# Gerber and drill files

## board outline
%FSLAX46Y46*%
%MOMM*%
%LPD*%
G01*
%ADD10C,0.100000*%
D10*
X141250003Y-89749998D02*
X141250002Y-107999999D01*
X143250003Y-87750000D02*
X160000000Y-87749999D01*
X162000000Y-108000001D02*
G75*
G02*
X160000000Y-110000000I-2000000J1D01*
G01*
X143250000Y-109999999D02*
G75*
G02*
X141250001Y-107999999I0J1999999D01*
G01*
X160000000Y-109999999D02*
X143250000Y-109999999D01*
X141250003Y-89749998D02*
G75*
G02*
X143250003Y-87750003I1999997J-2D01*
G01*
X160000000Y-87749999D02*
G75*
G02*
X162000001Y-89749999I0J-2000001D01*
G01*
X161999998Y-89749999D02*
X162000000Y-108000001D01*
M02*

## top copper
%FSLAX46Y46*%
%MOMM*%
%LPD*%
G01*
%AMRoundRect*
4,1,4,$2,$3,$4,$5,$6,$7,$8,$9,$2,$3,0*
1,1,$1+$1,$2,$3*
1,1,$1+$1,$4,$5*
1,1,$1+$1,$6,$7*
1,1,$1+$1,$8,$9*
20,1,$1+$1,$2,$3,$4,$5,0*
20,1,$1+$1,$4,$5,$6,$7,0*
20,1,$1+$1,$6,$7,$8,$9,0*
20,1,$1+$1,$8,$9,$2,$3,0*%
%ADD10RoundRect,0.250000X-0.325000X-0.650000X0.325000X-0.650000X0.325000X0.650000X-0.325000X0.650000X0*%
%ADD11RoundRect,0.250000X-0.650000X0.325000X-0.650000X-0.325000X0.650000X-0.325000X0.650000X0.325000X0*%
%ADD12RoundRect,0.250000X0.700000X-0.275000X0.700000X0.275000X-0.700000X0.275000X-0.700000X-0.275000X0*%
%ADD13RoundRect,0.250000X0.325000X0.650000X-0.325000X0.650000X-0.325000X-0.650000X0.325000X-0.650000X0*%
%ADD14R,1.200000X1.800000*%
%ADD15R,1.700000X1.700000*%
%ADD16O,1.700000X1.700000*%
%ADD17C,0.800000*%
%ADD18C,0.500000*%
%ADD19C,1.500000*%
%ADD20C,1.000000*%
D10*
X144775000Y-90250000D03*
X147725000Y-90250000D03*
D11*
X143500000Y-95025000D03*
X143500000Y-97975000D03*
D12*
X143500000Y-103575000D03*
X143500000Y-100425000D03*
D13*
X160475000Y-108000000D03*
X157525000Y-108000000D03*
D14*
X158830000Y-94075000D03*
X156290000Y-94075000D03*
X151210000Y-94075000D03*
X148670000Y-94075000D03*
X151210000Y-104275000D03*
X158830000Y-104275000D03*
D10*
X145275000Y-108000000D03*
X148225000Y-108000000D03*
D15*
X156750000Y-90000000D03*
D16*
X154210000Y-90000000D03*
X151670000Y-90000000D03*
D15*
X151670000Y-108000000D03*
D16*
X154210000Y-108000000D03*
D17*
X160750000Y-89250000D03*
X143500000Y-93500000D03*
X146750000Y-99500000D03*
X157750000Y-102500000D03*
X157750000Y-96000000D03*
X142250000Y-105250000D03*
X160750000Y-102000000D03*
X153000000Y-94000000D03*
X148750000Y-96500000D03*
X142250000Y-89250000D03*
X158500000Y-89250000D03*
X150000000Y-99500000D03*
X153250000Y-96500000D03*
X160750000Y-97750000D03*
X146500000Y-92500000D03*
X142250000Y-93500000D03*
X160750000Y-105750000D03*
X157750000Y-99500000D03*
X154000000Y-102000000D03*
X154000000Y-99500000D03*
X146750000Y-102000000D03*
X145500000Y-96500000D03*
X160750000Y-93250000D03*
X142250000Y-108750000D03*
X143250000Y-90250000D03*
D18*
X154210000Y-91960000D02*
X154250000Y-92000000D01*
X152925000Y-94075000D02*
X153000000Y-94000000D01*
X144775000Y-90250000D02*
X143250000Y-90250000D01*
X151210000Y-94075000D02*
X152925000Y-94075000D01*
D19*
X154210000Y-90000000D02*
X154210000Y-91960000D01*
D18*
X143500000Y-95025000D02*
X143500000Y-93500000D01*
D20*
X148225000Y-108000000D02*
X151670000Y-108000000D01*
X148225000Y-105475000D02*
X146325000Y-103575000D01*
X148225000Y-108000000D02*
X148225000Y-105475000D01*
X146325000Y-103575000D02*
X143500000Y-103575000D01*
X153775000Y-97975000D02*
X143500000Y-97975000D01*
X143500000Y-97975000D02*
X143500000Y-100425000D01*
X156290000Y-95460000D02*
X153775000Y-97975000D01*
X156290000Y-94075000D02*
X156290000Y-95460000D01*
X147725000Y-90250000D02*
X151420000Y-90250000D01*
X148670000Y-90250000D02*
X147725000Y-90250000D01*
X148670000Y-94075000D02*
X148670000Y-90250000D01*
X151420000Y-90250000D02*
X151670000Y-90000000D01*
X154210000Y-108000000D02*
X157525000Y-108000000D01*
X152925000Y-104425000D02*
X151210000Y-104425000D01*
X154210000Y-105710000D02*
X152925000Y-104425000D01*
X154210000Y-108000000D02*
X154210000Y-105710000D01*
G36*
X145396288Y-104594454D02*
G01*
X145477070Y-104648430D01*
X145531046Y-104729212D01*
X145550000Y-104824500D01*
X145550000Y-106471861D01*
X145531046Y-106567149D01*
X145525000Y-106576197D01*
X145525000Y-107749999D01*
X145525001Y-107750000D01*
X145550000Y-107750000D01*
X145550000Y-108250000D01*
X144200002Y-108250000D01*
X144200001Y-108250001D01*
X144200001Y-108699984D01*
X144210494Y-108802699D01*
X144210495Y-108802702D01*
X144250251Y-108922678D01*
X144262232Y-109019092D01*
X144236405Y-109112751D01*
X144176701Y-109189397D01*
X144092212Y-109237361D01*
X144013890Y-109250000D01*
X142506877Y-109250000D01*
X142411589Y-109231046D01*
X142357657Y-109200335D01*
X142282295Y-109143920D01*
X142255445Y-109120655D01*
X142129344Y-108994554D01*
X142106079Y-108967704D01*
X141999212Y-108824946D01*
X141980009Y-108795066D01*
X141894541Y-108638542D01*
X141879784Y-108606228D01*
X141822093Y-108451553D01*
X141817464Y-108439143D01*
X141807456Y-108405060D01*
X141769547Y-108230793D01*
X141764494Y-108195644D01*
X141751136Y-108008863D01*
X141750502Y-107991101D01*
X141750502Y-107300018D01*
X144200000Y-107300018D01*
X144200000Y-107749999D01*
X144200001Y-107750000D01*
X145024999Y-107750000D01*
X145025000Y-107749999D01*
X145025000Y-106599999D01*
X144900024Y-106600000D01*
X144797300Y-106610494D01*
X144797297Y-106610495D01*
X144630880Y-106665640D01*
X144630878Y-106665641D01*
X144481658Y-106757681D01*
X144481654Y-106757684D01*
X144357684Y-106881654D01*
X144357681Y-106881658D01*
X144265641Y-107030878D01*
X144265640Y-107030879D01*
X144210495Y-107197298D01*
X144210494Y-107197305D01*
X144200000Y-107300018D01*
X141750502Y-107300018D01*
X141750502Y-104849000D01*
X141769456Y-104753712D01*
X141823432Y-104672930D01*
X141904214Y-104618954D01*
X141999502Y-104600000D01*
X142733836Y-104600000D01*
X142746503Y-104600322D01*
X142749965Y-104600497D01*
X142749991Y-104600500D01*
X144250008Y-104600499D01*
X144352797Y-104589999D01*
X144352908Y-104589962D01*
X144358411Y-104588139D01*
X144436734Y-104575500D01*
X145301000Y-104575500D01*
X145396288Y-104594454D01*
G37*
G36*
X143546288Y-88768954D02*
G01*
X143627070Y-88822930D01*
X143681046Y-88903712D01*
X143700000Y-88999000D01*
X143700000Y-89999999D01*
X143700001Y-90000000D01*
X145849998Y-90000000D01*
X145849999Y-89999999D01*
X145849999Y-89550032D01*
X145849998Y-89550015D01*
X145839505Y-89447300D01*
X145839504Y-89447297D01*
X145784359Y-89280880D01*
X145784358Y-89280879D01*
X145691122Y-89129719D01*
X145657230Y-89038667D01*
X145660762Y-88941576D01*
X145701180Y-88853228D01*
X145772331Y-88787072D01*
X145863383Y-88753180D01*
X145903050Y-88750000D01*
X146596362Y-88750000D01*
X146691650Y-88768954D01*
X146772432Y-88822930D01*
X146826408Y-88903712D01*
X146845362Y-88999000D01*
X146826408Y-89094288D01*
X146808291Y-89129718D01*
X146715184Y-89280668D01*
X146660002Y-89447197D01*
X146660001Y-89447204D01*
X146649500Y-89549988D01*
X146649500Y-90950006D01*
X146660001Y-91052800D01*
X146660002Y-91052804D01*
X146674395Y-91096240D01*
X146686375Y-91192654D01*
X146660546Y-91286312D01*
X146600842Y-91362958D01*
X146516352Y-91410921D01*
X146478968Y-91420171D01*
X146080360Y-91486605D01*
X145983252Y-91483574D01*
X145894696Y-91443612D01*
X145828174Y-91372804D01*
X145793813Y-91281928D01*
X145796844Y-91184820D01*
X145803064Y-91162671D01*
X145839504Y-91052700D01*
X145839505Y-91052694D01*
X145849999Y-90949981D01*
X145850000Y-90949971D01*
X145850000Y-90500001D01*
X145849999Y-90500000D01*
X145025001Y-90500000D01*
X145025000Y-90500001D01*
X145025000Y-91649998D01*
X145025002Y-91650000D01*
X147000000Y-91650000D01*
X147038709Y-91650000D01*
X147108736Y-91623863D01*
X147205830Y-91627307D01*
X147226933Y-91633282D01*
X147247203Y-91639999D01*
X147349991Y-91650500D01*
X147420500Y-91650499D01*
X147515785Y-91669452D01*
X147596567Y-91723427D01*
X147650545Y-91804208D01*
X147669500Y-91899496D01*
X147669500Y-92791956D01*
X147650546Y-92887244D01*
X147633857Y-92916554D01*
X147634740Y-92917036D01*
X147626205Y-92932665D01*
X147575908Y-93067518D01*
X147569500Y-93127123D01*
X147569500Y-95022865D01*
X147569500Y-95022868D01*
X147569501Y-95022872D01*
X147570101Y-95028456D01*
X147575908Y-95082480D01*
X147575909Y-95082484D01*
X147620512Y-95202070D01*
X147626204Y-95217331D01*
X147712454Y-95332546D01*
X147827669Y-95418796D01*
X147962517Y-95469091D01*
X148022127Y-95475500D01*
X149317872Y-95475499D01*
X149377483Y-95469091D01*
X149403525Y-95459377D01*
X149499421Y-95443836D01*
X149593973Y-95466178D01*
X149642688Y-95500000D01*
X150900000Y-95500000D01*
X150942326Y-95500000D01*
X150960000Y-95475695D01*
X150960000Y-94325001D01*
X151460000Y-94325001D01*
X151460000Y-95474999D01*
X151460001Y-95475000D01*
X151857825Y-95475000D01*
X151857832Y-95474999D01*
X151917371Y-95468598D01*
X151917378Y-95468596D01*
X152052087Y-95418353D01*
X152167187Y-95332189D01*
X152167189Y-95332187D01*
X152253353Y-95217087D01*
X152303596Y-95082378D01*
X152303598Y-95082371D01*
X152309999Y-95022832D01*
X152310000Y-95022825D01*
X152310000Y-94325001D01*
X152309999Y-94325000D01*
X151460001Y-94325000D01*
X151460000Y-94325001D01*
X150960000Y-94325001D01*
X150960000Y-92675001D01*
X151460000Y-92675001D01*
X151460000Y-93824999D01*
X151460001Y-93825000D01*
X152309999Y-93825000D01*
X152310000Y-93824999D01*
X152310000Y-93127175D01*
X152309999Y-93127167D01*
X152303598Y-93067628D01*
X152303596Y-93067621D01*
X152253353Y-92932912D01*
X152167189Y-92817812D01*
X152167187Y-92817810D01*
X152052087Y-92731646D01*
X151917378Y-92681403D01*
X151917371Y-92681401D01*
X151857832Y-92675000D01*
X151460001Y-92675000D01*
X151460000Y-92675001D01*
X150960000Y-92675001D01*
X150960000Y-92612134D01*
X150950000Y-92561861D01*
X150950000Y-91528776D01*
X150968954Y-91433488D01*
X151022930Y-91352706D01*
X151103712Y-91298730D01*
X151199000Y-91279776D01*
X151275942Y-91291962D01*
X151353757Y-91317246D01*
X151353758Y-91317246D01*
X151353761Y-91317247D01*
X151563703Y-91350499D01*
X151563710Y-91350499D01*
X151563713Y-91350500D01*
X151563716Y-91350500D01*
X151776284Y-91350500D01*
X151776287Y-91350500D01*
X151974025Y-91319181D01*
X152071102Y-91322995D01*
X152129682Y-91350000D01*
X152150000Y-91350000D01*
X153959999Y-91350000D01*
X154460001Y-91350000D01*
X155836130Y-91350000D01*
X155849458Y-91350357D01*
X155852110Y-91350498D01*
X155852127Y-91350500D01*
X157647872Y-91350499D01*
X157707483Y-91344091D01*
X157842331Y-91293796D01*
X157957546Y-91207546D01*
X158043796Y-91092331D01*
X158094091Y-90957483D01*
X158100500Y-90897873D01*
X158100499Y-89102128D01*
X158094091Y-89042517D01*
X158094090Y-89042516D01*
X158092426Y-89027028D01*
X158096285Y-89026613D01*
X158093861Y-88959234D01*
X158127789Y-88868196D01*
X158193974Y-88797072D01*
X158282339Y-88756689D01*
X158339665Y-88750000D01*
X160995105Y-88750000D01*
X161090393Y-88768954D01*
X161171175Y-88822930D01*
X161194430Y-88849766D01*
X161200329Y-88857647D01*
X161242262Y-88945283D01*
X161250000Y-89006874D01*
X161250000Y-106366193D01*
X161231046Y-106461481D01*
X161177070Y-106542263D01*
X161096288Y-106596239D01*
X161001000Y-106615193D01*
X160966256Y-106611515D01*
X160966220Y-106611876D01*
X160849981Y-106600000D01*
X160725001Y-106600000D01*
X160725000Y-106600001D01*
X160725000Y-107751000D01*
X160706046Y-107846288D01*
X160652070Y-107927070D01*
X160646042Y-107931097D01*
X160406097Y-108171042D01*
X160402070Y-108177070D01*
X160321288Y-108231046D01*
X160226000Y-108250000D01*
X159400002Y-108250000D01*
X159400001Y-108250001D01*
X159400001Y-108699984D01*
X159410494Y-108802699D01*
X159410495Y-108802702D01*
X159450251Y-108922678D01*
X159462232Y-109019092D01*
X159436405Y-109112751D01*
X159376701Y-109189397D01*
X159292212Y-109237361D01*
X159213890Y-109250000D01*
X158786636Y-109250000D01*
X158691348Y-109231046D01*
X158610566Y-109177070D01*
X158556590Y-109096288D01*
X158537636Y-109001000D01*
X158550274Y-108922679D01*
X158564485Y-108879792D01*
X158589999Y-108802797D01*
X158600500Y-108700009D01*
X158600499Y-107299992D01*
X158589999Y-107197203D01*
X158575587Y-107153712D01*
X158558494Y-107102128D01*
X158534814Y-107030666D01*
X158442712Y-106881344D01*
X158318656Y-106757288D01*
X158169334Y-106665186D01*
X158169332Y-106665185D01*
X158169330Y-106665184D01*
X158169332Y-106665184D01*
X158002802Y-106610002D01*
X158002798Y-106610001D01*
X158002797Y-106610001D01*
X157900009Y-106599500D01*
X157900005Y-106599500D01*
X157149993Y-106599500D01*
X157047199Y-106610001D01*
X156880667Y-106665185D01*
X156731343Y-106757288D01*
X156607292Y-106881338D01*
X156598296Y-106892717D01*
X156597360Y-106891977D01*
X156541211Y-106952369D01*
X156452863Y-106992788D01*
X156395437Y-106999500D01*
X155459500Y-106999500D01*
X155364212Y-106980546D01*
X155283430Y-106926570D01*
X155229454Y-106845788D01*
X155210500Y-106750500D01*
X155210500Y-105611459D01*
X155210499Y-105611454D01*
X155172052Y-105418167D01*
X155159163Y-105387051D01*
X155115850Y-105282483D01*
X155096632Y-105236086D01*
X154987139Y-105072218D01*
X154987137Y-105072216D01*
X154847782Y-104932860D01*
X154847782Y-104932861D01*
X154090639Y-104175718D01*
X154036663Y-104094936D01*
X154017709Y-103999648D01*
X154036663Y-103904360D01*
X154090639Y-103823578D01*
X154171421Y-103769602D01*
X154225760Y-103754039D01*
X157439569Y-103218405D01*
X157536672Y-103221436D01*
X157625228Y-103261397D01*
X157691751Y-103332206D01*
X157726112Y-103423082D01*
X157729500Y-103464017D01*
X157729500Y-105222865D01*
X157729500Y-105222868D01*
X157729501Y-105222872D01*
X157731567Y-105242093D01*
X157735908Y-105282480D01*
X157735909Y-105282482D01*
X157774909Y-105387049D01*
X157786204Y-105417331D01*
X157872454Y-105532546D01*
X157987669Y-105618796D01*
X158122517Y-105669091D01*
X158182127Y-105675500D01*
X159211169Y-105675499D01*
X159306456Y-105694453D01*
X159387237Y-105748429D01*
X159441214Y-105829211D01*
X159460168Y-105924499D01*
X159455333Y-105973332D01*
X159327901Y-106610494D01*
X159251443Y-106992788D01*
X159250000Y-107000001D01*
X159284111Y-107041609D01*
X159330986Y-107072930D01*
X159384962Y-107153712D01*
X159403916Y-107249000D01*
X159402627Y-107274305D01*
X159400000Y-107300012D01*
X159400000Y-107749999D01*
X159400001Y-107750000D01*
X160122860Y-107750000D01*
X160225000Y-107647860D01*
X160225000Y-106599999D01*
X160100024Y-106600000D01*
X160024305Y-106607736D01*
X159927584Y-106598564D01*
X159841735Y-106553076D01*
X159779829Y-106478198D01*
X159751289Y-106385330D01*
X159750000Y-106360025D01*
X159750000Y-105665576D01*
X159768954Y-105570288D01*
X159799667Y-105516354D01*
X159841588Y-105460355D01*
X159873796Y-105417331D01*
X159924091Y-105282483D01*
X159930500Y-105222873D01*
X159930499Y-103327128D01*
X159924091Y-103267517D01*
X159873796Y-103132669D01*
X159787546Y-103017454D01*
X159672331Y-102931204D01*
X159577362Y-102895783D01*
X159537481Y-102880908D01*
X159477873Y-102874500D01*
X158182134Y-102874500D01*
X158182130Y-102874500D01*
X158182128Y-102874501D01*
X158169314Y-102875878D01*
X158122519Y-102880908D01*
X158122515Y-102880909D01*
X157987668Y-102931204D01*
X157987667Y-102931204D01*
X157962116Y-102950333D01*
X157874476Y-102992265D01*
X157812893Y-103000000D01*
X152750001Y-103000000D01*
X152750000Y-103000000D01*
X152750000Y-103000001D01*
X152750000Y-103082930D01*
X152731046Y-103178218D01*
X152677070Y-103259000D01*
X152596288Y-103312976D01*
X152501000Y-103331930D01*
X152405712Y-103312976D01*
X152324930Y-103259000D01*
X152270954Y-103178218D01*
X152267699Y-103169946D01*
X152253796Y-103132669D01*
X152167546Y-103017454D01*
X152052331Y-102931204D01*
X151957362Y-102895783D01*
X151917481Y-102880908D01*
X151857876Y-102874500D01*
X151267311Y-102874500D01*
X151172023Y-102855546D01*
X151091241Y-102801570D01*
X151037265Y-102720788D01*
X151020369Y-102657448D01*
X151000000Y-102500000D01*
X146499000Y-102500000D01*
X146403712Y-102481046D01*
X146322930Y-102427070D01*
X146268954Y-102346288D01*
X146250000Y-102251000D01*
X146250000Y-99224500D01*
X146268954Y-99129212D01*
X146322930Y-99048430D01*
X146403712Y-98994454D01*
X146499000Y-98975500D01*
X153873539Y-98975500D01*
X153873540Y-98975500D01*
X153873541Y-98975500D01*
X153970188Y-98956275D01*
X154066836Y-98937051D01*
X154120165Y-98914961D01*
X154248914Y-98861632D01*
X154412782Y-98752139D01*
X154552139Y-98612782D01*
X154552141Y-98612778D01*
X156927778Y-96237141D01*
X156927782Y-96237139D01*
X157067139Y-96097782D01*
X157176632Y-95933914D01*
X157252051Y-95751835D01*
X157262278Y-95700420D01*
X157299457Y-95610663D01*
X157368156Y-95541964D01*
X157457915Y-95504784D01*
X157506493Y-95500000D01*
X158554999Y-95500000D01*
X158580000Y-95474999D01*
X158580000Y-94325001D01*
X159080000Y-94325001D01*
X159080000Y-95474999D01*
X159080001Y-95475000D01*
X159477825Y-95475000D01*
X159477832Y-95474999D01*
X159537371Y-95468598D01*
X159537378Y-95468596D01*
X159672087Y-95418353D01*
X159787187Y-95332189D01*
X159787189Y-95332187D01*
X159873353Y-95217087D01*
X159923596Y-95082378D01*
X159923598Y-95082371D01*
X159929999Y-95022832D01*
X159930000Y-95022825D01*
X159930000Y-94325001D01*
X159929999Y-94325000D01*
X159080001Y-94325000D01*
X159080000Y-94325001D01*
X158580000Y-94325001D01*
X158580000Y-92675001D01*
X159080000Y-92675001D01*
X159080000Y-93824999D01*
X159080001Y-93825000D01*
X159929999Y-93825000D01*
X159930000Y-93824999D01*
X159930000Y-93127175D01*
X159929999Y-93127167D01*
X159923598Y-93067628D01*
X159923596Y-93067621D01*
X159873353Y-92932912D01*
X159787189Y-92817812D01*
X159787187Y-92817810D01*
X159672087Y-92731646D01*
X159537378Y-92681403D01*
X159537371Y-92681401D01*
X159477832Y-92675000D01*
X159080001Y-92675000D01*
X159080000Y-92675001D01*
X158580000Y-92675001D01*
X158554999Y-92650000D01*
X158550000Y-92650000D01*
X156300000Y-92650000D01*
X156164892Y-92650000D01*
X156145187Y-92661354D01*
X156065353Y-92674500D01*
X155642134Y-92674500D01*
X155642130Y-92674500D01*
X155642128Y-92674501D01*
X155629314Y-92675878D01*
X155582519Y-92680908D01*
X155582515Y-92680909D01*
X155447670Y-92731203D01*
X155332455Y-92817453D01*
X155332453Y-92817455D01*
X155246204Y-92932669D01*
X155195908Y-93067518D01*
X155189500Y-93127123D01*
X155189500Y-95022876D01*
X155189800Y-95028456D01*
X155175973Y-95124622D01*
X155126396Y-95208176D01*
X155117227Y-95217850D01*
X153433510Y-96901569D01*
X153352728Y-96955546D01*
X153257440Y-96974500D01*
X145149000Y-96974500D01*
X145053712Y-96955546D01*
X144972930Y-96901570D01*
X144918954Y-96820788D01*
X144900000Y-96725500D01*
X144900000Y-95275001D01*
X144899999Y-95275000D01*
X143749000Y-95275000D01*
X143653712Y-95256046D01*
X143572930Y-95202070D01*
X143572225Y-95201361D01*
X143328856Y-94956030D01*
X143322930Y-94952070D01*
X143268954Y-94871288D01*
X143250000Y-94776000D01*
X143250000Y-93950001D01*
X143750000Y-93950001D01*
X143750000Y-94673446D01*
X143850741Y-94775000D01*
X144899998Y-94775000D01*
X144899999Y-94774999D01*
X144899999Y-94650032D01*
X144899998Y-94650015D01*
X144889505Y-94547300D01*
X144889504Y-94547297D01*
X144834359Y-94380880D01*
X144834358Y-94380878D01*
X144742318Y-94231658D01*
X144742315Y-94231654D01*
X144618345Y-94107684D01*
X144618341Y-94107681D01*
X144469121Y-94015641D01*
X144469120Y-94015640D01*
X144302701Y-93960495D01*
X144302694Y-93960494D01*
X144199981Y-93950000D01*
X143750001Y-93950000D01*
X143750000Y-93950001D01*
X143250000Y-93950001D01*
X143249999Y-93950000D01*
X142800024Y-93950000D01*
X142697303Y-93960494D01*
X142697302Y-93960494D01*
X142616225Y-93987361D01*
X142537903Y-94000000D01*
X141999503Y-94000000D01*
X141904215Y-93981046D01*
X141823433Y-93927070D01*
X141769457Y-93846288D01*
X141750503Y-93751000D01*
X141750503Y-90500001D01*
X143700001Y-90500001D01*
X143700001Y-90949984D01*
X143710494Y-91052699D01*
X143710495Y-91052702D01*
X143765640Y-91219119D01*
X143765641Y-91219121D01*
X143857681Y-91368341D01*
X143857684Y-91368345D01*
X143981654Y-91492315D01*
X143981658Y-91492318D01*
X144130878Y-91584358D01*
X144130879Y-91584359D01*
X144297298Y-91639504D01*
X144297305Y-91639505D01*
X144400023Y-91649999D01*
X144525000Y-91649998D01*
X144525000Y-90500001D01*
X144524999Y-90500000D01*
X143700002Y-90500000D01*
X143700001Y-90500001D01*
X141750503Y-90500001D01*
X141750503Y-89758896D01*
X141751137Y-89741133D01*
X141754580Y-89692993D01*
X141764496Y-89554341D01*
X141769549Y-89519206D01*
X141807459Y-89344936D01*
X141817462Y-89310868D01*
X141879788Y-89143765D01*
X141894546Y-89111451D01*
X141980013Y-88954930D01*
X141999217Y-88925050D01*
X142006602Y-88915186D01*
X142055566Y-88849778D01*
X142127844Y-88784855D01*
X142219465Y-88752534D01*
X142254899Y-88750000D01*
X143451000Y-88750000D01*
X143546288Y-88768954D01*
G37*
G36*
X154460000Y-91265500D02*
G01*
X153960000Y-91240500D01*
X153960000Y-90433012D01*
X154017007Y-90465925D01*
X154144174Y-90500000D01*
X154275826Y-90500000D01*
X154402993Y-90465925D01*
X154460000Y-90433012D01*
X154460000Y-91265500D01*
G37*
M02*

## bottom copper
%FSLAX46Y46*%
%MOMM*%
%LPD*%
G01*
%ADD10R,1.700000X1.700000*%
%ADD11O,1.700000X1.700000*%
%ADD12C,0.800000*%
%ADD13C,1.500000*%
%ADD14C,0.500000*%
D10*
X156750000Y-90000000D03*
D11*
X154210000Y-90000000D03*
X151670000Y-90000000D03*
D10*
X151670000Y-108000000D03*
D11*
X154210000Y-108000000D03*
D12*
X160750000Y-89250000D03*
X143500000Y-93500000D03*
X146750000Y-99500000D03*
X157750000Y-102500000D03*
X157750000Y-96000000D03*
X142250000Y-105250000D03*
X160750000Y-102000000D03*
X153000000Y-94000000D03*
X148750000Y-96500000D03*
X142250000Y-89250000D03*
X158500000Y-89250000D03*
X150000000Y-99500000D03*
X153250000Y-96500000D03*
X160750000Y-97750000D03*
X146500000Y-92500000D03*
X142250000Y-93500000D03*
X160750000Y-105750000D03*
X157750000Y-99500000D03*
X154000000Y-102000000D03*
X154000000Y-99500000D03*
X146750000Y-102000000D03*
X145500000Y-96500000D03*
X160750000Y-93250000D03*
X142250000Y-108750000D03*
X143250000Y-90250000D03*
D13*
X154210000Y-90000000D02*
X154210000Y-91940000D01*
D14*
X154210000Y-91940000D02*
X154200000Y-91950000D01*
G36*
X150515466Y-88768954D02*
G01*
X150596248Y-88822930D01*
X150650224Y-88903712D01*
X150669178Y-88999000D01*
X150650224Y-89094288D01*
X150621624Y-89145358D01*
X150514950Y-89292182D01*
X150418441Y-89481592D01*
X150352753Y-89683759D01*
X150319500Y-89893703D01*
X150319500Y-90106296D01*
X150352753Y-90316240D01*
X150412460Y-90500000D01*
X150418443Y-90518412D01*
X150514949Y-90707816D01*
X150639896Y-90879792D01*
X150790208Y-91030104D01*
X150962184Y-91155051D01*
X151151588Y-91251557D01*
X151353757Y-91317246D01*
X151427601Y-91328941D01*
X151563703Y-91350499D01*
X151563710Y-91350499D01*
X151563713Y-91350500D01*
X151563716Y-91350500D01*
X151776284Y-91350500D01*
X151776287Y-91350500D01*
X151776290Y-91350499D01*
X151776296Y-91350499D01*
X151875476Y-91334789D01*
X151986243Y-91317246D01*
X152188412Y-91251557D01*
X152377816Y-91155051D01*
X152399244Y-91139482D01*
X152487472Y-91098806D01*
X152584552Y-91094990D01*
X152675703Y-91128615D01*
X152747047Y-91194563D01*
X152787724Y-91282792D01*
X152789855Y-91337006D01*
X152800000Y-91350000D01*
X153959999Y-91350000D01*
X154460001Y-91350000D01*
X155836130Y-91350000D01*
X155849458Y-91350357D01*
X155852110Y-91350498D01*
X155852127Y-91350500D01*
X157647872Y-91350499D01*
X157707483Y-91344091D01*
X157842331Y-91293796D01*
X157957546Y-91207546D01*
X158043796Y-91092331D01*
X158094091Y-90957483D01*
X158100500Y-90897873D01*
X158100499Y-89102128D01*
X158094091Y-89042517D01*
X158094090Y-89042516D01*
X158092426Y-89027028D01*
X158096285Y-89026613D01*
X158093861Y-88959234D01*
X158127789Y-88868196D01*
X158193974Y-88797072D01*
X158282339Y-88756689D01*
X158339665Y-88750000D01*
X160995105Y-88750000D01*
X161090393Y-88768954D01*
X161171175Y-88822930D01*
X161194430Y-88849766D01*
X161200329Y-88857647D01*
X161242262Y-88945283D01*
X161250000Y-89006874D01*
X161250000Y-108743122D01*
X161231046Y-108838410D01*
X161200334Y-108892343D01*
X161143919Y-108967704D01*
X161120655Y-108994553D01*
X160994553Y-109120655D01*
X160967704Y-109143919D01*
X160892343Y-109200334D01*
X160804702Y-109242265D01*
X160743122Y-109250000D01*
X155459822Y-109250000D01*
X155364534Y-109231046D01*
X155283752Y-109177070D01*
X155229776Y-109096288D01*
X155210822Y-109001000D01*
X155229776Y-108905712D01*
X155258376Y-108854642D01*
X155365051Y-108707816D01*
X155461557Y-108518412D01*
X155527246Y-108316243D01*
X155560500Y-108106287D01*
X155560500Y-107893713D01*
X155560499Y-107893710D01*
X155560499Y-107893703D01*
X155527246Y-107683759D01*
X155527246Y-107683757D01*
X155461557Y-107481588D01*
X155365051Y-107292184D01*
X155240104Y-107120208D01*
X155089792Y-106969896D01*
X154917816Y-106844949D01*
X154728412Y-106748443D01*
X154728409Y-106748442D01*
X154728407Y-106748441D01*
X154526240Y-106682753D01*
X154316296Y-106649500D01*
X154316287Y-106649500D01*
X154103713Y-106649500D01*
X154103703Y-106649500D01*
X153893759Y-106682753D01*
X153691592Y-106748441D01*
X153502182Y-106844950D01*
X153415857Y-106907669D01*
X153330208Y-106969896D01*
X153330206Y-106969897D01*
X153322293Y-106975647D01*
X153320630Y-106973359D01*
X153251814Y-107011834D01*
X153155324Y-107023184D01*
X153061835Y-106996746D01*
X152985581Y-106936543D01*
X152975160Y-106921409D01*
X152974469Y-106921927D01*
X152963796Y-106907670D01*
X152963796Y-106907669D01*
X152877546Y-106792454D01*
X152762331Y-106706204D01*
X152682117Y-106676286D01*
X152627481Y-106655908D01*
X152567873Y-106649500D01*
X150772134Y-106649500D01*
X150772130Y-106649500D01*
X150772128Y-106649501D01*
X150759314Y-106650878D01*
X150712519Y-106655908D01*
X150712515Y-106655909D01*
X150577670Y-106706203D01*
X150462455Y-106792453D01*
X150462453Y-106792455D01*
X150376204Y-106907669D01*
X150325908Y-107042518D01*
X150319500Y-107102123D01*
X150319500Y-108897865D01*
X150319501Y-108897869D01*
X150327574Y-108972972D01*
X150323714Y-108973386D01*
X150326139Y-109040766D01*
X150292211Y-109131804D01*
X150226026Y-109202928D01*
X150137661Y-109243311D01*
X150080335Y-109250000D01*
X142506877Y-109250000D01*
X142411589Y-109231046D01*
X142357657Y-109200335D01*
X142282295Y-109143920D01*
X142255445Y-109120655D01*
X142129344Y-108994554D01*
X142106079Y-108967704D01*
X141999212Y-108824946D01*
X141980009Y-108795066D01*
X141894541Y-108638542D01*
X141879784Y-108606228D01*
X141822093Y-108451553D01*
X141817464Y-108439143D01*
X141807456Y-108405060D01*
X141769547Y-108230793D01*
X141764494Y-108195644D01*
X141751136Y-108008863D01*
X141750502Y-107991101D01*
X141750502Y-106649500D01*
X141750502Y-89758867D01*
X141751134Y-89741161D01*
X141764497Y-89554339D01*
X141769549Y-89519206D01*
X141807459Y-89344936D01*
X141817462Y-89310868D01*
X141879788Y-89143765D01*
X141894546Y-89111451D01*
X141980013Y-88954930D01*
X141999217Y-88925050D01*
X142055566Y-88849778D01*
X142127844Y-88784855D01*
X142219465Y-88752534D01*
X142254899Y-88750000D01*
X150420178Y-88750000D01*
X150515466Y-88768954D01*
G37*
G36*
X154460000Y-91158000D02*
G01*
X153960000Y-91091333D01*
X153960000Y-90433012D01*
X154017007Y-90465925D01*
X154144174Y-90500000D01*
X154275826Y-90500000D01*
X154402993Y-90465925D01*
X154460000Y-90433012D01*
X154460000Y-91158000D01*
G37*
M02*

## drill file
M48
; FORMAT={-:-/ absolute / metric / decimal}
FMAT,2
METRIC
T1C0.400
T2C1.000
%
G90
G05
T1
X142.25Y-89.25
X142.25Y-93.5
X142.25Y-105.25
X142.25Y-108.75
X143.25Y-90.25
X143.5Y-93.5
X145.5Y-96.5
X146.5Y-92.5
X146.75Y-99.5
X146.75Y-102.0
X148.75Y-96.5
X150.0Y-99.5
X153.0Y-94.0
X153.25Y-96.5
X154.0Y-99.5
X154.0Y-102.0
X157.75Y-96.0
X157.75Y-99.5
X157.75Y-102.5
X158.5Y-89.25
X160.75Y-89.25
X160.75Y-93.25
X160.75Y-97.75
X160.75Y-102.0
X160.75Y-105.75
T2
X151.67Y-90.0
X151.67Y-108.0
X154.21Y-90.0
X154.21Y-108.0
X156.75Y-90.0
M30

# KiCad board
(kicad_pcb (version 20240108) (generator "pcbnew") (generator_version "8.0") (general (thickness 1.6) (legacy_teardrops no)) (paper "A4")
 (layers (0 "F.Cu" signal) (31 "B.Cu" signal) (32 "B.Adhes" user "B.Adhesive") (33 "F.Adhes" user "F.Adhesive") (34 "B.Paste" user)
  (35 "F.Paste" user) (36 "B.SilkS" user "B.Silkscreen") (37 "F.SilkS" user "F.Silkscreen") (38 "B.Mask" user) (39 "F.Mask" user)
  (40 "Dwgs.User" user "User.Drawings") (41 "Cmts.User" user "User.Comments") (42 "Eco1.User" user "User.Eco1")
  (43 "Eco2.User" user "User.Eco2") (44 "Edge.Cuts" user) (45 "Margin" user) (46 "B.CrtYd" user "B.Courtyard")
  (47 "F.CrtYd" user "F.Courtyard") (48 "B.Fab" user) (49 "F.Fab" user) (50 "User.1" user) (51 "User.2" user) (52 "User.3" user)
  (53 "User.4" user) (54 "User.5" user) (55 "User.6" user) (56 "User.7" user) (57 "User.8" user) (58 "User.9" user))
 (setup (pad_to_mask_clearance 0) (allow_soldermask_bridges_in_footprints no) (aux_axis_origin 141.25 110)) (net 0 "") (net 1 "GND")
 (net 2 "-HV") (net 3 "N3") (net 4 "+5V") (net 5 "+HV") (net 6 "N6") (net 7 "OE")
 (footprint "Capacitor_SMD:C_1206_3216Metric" (layer "F.Cu") (at 146.25 90.25)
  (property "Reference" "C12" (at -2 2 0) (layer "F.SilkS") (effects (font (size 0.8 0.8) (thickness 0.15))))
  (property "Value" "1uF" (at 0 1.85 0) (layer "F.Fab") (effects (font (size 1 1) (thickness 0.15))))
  (pad "1" smd roundrect (at -1.475 0) (size 1.15 1.8) (layers "F.Cu" "F.Paste" "F.Mask") (roundrect_rratio 0.2173913043) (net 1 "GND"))
  (pad "2" smd roundrect (at 1.475 0) (size 1.15 1.8) (layers "F.Cu" "F.Paste" "F.Mask") (roundrect_rratio 0.2173913043) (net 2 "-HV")))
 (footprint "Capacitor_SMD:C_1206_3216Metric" (layer "F.Cu") (at 143.5 96.5 -90)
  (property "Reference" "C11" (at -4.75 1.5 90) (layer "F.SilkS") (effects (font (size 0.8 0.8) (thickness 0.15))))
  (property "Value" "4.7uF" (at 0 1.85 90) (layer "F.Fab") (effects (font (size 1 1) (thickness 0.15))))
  (pad "1" smd roundrect (at -1.475 0 270) (size 1.15 1.8) (layers "F.Cu" "F.Paste" "F.Mask") (roundrect_rratio 0.2173913043) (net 1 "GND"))
  (pad "2" smd roundrect (at 1.475 0 270) (size 1.15 1.8) (layers "F.Cu" "F.Paste" "F.Mask") (roundrect_rratio 0.2173913043) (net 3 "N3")))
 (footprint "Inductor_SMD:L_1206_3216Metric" (layer "F.Cu") (at 143.5 102 90)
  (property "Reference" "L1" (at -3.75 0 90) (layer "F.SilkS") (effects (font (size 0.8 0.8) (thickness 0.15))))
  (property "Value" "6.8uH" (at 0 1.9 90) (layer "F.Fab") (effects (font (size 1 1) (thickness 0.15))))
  (pad "1" smd roundrect (at -1.575 0 90) (size 1.05 1.9) (layers "F.Cu" "F.Paste" "F.Mask") (roundrect_rratio 0.2380952381) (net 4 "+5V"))
  (pad "2" smd roundrect (at 1.575 0 90) (size 1.05 1.9) (layers "F.Cu" "F.Paste" "F.Mask") (roundrect_rratio 0.2380952381) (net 3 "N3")))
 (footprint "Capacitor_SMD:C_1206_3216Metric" (layer "F.Cu") (at 159 108 180)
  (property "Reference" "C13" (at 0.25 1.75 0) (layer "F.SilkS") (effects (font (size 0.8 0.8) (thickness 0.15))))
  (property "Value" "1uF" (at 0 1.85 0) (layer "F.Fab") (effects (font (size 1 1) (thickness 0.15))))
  (pad "1" smd roundrect (at -1.475 0 180) (size 1.15 1.8) (layers "F.Cu" "F.Paste" "F.Mask") (roundrect_rratio 0.2173913043) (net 1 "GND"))
  (pad "2" smd roundrect (at 1.475 0 180) (size 1.15 1.8) (layers "F.Cu" "F.Paste" "F.Mask") (roundrect_rratio 0.2173913043) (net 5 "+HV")))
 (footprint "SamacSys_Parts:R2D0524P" (layer "F.Cu") (at 153.75 99.175 180)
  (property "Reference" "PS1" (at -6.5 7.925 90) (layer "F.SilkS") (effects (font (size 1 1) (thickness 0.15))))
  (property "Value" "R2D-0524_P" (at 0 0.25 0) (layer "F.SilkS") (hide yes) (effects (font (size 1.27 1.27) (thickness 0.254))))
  (pad "1" smd rect (at -5.08 5.1 180) (size 1.2 1.8) (layers "F.Cu" "F.Paste" "F.Mask") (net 1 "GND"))
  (pad "2" smd rect (at -2.54 5.1 180) (size 1.2 1.8) (layers "F.Cu" "F.Paste" "F.Mask") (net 3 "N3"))
  (pad "4" smd rect (at 2.54 5.1 180) (size 1.2 1.8) (layers "F.Cu" "F.Paste" "F.Mask") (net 1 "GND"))
  (pad "5" smd rect (at 5.08 5.1 180) (size 1.2 1.8) (layers "F.Cu" "F.Paste" "F.Mask") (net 2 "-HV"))
  (pad "7" smd rect (at 2.54 -5.1 180) (size 1.2 1.8) (layers "F.Cu" "F.Paste" "F.Mask") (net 5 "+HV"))
  (pad "10" smd rect (at -5.08 -5.1 180) (size 1.2 1.8) (layers "F.Cu" "F.Paste" "F.Mask") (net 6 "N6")))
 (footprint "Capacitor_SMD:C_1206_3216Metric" (layer "F.Cu") (at 146.75 108)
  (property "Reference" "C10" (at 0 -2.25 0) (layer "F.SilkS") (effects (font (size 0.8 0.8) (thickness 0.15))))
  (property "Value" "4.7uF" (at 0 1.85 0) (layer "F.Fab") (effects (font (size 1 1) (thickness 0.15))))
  (pad "1" smd roundrect (at -1.475 0) (size 1.15 1.8) (layers "F.Cu" "F.Paste" "F.Mask") (roundrect_rratio 0.2173913043) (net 1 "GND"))
  (pad "2" smd roundrect (at 1.475 0) (size 1.15 1.8) (layers "F.Cu" "F.Paste" "F.Mask") (roundrect_rratio 0.2173913043) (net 4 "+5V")))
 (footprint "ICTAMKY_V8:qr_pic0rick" (layer "B.Cu") (at 152 98 180)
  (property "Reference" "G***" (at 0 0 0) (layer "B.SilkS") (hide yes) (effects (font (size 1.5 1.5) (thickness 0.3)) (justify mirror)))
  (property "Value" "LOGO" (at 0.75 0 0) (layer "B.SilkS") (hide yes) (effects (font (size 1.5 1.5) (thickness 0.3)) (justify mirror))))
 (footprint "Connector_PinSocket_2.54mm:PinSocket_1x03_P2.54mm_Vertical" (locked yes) (layer "B.Cu") (at 156.75 90 90)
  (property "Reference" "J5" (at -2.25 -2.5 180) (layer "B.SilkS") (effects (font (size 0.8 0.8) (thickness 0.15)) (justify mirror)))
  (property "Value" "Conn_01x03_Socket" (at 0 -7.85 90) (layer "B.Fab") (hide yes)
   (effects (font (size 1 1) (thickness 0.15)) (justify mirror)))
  (pad "1" thru_hole rect (at 0 0 90) (size 1.7 1.7) (drill 1) (layers "*.Cu" "*.Mask") (remove_unused_layers no) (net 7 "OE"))
  (pad "2" thru_hole oval (at 0 -2.54 90) (size 1.7 1.7) (drill 1) (layers "*.Cu" "*.Mask") (remove_unused_layers no) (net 1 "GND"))
  (pad "3" thru_hole oval (at 0 -5.08 90) (size 1.7 1.7) (drill 1) (layers "*.Cu" "*.Mask") (remove_unused_layers no) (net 2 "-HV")))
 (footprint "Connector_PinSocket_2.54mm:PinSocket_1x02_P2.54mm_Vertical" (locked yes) (layer "B.Cu") (at 151.67 108 -90)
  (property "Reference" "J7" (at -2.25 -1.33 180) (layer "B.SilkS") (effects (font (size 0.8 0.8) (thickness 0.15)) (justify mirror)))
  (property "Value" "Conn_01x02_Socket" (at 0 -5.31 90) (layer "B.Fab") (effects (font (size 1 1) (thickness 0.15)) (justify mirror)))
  (pad "1" thru_hole rect (at 0 0 270) (size 1.7 1.7) (drill 1) (layers "*.Cu" "*.Mask") (remove_unused_layers no) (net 4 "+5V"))
  (pad "2" thru_hole oval (at 0 -2.54 270) (size 1.7 1.7) (drill 1) (layers "*.Cu" "*.Mask") (remove_unused_layers no) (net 5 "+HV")))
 (gr_line (start 141.250003 89.749998) (end 141.250002 107.999999) (stroke (width 0.1) (type default)) (layer "Edge.Cuts"))
 (gr_line (start 143.250003 87.75) (end 160 87.749999) (stroke (width 0.1) (type default)) (layer "Edge.Cuts"))
 (gr_arc (start 162 108.000001) (mid 161.414213 109.414213) (end 160 109.999999) (stroke (width 0.1) (type default)) (layer "Edge.Cuts"))
 (gr_arc (start 143.25 109.999999) (mid 141.835786 109.414213) (end 141.250002 107.999999) (stroke (width 0.1) (type default))
  (layer "Edge.Cuts"))
 (gr_line (start 160 109.999999) (end 143.25 109.999999) (stroke (width 0.1) (type default)) (layer "Edge.Cuts"))
 (gr_arc (start 141.250003 89.749998) (mid 141.83579 88.335786) (end 143.250003 87.75) (stroke (width 0.1) (type default))
  (layer "Edge.Cuts"))
 (gr_arc (start 160 87.749999) (mid 161.414214 88.335785) (end 161.999998 89.749999) (stroke (width 0.1) (type default)) (layer "Edge.Cuts"))
 (gr_line (start 161.999998 89.749999) (end 162 108.000001) (stroke (width 0.1) (type default)) (layer "Edge.Cuts"))
 (segment (start 154.21 91.96) (end 154.25 92) (width 0.5) (layer "F.Cu") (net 1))
 (segment (start 152.925 94.075) (end 153 94) (width 0.5) (layer "F.Cu") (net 1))
 (segment (start 144.775 90.25) (end 143.25 90.25) (width 0.5) (layer "F.Cu") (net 1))
 (segment (start 151.21 94.075) (end 152.925 94.075) (width 0.5) (layer "F.Cu") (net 1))
 (segment (start 154.21 90) (end 154.21 91.96) (width 1.5) (layer "F.Cu") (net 1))
 (segment (start 143.5 95.025) (end 143.5 93.5) (width 0.5) (layer "F.Cu") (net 1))
 (via (at 160.75 89.25) (size 0.8) (drill 0.4) (layers "F.Cu" "B.Cu") (free yes) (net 1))
 (via (at 143.5 93.5) (size 0.8) (drill 0.4) (layers "F.Cu" "B.Cu") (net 1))
 (via (at 146.75 99.5) (size 0.8) (drill 0.4) (layers "F.Cu" "B.Cu") (free yes) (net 1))
 (via (at 157.75 102.5) (size 0.8) (drill 0.4) (layers "F.Cu" "B.Cu") (free yes) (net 1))
 (via (at 157.75 96) (size 0.8) (drill 0.4) (layers "F.Cu" "B.Cu") (free yes) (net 1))
 (via (at 142.25 105.25) (size 0.8) (drill 0.4) (layers "F.Cu" "B.Cu") (free yes) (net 1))
 (via (at 160.75 102) (size 0.8) (drill 0.4) (layers "F.Cu" "B.Cu") (free yes) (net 1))
 (via (at 153 94) (size 0.8) (drill 0.4) (layers "F.Cu" "B.Cu") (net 1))
 (via (at 148.75 96.5) (size 0.8) (drill 0.4) (layers "F.Cu" "B.Cu") (free yes) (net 1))
 (via (at 142.25 89.25) (size 0.8) (drill 0.4) (layers "F.Cu" "B.Cu") (free yes) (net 1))
 (via (at 158.5 89.25) (size 0.8) (drill 0.4) (layers "F.Cu" "B.Cu") (free yes) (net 1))
 (via (at 150 99.5) (size 0.8) (drill 0.4) (layers "F.Cu" "B.Cu") (free yes) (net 1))
 (via (at 153.25 96.5) (size 0.8) (drill 0.4) (layers "F.Cu" "B.Cu") (free yes) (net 1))
 (via (at 160.75 97.75) (size 0.8) (drill 0.4) (layers "F.Cu" "B.Cu") (free yes) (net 1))
 (via (at 146.5 92.5) (size 0.8) (drill 0.4) (layers "F.Cu" "B.Cu") (free yes) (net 1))
 (via (at 142.25 93.5) (size 0.8) (drill 0.4) (layers "F.Cu" "B.Cu") (free yes) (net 1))
 (via (at 160.75 105.75) (size 0.8) (drill 0.4) (layers "F.Cu" "B.Cu") (free yes) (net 1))
 (via (at 157.75 99.5) (size 0.8) (drill 0.4) (layers "F.Cu" "B.Cu") (free yes) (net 1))
 (via (at 154 102) (size 0.8) (drill 0.4) (layers "F.Cu" "B.Cu") (free yes) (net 1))
 (via (at 154 99.5) (size 0.8) (drill 0.4) (layers "F.Cu" "B.Cu") (free yes) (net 1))
 (via (at 146.75 102) (size 0.8) (drill 0.4) (layers "F.Cu" "B.Cu") (free yes) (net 1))
 (via (at 145.5 96.5) (size 0.8) (drill 0.4) (layers "F.Cu" "B.Cu") (free yes) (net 1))
 (via (at 160.75 93.25) (size 0.8) (drill 0.4) (layers "F.Cu" "B.Cu") (free yes) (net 1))
 (via (at 142.25 108.75) (size 0.8) (drill 0.4) (layers "F.Cu" "B.Cu") (free yes) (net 1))
 (via (at 143.25 90.25) (size 0.8) (drill 0.4) (layers "F.Cu" "B.Cu") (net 1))
 (segment (start 154.21 90) (end 154.21 91.94) (width 1.5) (layer "B.Cu") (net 1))
 (segment (start 154.21 91.94) (end 154.2 91.95) (width 0.5) (layer "B.Cu") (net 1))
 (segment (start 148.225 108) (end 151.67 108) (width 1) (layer "F.Cu") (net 4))
 (segment (start 148.225 105.475) (end 146.325 103.575) (width 1) (layer "F.Cu") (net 4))
 (segment (start 148.225 108) (end 148.225 105.475) (width 1) (layer "F.Cu") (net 4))
 (segment (start 146.325 103.575) (end 143.5 103.575) (width 1) (layer "F.Cu") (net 4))
 (segment (start 153.775 97.975) (end 143.5 97.975) (width 1) (layer "F.Cu") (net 3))
 (segment (start 143.5 97.975) (end 143.5 100.425) (width 1) (layer "F.Cu") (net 3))
 (segment (start 156.29 95.46) (end 153.775 97.975) (width 1) (layer "F.Cu") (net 3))
 (segment (start 156.29 94.075) (end 156.29 95.46) (width 1) (layer "F.Cu") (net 3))
 (segment (start 147.725 90.25) (end 151.42 90.25) (width 1) (layer "F.Cu") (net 2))
 (segment (start 148.67 90.25) (end 147.725 90.25) (width 1) (layer "F.Cu") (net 2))
 (segment (start 148.67 94.075) (end 148.67 90.25) (width 1) (layer "F.Cu") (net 2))
 (segment (start 151.42 90.25) (end 151.67 90) (width 1) (layer "F.Cu") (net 2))
 (segment (start 154.21 108) (end 157.525 108) (width 1) (layer "F.Cu") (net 5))
 (segment (start 152.925 104.425) (end 151.21 104.425) (width 1) (layer "F.Cu") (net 5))
 (segment (start 154.21 105.71) (end 152.925 104.425) (width 1) (layer "F.Cu") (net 5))
 (segment (start 154.21 108) (end 154.21 105.71) (width 1) (layer "F.Cu") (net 5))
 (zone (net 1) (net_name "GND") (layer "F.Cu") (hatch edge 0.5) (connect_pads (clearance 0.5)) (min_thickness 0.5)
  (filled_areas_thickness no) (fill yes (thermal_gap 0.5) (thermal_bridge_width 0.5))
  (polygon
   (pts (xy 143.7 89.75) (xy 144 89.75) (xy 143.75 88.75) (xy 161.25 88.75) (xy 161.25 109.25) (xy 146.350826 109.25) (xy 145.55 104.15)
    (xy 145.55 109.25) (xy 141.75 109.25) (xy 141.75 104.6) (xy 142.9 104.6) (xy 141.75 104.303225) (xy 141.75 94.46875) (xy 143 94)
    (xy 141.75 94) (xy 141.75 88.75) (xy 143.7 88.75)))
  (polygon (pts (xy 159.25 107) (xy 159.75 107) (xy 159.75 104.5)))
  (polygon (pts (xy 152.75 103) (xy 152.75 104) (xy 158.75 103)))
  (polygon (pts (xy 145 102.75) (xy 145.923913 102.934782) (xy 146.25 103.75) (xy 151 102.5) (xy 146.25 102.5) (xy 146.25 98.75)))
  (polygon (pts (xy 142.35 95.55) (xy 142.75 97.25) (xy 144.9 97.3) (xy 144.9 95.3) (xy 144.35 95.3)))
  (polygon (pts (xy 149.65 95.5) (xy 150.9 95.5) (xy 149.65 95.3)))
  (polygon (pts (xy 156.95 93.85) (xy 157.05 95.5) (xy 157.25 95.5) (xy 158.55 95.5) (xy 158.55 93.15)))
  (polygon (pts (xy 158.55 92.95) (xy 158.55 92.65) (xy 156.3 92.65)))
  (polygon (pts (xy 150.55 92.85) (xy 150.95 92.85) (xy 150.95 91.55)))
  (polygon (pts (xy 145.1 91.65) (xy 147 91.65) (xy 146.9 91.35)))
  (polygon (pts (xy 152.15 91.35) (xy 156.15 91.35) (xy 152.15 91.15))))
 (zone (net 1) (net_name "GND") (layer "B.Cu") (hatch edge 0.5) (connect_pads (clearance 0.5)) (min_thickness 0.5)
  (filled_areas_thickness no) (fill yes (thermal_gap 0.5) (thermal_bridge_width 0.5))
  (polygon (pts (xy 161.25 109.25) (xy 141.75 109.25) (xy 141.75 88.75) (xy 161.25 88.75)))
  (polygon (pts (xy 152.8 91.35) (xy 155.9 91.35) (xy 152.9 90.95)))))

